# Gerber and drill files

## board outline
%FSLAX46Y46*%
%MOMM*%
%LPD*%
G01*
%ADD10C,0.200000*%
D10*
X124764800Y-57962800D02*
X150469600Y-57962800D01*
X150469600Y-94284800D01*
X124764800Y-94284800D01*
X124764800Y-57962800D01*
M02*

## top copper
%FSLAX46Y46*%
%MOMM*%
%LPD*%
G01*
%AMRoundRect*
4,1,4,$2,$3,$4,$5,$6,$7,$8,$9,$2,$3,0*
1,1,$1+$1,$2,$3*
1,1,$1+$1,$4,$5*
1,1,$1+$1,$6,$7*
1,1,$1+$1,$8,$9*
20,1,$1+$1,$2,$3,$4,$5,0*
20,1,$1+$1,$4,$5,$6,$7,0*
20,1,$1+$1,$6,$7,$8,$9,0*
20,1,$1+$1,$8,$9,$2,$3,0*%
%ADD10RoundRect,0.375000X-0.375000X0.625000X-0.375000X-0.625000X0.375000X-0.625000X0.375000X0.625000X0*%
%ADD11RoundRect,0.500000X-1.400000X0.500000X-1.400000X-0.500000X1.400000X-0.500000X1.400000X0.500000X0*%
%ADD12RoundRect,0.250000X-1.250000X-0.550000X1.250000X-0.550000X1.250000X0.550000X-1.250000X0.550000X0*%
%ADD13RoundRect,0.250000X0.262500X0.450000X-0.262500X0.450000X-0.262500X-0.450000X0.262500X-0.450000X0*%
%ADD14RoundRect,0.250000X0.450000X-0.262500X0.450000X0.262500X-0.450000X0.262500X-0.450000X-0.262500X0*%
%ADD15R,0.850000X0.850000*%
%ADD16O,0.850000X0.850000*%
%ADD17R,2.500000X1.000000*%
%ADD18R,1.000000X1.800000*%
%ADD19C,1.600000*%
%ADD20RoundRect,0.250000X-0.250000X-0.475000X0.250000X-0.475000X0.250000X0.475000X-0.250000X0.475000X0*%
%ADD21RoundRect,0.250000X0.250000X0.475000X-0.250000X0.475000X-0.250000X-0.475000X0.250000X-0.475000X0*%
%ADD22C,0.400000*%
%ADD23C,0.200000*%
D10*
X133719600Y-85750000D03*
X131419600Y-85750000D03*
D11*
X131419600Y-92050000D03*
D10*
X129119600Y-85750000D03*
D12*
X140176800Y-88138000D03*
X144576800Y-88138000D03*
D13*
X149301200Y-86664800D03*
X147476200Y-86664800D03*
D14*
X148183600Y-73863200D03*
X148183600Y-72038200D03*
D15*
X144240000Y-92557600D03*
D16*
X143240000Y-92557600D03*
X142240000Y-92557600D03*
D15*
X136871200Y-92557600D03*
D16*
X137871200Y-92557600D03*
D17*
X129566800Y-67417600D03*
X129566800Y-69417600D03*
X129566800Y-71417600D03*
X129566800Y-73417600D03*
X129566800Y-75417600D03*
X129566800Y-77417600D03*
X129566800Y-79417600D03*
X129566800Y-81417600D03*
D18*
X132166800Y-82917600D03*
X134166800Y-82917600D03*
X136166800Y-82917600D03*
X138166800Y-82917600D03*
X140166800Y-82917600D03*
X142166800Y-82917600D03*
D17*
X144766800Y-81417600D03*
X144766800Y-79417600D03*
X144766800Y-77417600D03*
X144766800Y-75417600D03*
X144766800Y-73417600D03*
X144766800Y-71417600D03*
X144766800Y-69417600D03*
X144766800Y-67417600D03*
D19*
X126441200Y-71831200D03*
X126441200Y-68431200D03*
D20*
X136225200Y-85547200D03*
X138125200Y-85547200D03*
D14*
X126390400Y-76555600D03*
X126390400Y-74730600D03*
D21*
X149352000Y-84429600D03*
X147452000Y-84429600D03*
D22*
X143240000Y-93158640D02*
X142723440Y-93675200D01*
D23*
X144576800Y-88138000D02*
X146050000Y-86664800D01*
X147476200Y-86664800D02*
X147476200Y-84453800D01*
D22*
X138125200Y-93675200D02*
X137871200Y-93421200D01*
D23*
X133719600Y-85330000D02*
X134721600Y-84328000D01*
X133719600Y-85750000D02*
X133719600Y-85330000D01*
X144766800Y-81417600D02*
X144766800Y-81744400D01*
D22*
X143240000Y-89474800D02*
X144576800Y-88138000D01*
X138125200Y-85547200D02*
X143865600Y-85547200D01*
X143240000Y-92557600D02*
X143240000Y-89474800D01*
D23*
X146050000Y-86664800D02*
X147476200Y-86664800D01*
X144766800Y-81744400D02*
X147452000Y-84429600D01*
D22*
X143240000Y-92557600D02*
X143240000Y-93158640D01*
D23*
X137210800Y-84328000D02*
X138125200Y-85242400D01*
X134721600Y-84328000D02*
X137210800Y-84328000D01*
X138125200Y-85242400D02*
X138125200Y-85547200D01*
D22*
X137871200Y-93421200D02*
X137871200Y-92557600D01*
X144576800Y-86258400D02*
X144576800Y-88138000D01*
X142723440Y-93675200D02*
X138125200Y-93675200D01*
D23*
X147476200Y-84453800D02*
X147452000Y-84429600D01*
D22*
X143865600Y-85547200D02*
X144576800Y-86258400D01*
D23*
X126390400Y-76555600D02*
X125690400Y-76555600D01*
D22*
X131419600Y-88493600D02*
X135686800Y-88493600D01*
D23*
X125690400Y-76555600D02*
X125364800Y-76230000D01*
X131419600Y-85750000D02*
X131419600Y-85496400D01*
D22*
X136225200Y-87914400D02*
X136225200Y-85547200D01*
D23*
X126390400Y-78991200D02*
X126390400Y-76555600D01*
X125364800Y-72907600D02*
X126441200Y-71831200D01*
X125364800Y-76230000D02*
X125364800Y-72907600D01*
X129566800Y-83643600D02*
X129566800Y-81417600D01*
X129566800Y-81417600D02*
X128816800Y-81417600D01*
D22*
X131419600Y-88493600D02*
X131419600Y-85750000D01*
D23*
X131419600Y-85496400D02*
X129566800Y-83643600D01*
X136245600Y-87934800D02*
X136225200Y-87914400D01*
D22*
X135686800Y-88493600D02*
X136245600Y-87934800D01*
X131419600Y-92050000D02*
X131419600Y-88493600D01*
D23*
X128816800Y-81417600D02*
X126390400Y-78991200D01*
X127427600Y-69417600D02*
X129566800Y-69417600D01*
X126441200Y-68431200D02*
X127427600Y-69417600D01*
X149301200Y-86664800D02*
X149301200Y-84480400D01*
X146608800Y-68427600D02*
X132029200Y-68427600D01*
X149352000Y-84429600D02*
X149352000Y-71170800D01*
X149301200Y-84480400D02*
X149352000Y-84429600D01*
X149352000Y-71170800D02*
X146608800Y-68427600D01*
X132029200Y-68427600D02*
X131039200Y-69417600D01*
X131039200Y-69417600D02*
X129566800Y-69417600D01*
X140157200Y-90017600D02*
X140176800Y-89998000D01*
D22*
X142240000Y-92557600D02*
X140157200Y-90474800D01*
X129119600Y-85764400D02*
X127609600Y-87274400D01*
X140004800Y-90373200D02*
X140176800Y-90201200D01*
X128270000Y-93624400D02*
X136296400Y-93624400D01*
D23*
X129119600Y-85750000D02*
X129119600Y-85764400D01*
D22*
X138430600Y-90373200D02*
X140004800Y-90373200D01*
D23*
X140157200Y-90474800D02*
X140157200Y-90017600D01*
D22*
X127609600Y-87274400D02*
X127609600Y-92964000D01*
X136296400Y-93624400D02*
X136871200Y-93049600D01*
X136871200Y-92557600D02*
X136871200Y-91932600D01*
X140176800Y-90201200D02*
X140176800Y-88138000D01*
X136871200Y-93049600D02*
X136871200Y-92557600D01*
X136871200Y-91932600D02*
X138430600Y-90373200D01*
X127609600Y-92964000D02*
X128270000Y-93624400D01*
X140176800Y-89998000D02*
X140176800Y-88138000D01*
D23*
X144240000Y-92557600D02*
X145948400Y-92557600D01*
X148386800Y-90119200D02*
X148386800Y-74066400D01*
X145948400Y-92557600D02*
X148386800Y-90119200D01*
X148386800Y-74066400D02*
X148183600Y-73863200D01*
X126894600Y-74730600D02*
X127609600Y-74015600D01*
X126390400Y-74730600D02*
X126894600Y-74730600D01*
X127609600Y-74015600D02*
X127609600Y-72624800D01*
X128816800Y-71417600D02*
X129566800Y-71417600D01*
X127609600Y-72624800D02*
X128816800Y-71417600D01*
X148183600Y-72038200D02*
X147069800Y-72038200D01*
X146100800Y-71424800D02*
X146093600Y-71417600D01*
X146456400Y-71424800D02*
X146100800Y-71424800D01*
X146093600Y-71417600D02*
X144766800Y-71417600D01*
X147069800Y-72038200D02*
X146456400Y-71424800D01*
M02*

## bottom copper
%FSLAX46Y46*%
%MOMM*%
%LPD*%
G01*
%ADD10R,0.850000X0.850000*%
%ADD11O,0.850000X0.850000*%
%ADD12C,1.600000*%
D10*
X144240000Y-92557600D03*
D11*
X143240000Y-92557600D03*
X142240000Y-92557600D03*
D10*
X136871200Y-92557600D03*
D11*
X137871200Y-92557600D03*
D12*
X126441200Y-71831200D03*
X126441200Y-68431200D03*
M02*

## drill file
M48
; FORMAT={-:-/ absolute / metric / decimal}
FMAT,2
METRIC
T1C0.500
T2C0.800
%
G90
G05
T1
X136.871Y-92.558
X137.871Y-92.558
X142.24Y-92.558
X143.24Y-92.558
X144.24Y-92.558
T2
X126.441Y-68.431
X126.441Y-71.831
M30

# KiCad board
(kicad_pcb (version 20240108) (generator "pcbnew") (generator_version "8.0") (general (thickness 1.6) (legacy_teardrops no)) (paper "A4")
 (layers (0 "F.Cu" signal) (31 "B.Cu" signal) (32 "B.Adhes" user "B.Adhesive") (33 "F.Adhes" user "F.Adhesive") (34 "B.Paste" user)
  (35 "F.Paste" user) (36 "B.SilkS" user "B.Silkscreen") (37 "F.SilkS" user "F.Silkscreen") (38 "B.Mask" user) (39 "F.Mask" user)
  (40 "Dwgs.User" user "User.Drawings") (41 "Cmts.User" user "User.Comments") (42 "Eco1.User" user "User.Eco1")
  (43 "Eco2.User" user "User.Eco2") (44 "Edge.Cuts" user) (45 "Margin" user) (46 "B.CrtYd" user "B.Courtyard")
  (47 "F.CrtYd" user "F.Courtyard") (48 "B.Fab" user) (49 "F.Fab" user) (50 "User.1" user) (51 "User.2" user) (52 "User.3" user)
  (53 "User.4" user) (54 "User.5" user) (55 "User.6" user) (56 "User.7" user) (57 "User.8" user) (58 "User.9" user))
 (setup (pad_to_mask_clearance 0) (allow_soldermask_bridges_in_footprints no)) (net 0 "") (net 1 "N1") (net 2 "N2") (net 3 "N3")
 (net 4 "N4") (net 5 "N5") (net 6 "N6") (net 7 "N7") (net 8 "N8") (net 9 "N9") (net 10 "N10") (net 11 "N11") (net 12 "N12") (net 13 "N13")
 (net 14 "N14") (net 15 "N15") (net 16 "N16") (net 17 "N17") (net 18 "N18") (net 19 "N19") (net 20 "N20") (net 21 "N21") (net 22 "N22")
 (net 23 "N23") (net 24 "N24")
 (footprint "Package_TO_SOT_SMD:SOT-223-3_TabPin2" (layer "F.Cu") (at 131.4196 88.9 -90)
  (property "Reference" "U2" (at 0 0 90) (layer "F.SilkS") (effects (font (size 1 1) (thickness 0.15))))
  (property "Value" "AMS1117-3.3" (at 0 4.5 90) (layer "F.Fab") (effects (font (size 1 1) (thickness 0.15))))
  (pad "1" smd roundrect (at -3.15 -2.3 270) (size 2 1.5) (layers "F.Cu" "F.Paste" "F.Mask") (roundrect_rratio 0.25) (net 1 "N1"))
  (pad "2" smd roundrect (at -3.15 0 270) (size 2 1.5) (layers "F.Cu" "F.Paste" "F.Mask") (roundrect_rratio 0.25) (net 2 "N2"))
  (pad "2" smd roundrect (at 3.15 0 270) (size 2 3.8) (layers "F.Cu" "F.Paste" "F.Mask") (roundrect_rratio 0.25) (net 2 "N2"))
  (pad "3" smd roundrect (at -3.15 2.3 270) (size 2 1.5) (layers "F.Cu" "F.Paste" "F.Mask") (roundrect_rratio 0.25) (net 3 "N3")))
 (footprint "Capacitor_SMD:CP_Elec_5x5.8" (layer "F.Cu") (at 142.3768 88.138)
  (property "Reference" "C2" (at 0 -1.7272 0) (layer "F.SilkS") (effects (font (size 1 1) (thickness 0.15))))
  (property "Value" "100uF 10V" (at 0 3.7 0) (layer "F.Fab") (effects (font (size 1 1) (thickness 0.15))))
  (pad "1" smd roundrect (at -2.2 0) (size 3 1.6) (layers "F.Cu" "F.Paste" "F.Mask") (roundrect_rratio 0.15625) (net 3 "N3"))
  (pad "2" smd roundrect (at 2.2 0) (size 3 1.6) (layers "F.Cu" "F.Paste" "F.Mask") (roundrect_rratio 0.15625) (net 1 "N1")))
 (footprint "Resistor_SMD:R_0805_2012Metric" (layer "F.Cu") (at 148.3887 86.6648 180)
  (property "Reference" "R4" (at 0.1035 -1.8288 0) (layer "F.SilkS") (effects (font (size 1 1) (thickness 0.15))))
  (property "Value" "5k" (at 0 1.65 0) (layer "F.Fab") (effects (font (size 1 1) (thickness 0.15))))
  (pad "1" smd roundrect (at -0.9125 0 180) (size 1.025 1.4) (layers "F.Cu" "F.Paste" "F.Mask") (roundrect_rratio 0.243902) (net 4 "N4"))
  (pad "2" smd roundrect (at 0.9125 0 180) (size 1.025 1.4) (layers "F.Cu" "F.Paste" "F.Mask") (roundrect_rratio 0.243902) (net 1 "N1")))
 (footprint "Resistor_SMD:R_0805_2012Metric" (layer "F.Cu") (at 148.1836 72.9507 90)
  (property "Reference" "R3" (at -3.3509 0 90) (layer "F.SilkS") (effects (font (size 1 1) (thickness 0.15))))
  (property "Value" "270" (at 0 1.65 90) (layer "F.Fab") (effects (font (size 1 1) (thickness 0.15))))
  (pad "1" smd roundrect (at -0.9125 0 90) (size 1.025 1.4) (layers "F.Cu" "F.Paste" "F.Mask") (roundrect_rratio 0.243902) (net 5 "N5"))
  (pad "2" smd roundrect (at 0.9125 0 90) (size 1.025 1.4) (layers "F.Cu" "F.Paste" "F.Mask") (roundrect_rratio 0.243902) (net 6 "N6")))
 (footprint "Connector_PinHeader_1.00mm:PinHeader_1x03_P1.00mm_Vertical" (layer "F.Cu") (at 144.24 92.5576 -90)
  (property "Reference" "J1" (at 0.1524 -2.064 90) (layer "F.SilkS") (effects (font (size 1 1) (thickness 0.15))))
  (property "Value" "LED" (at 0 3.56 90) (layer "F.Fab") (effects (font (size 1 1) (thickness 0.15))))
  (pad "1" thru_hole rect (at 0 0 270) (size 0.85 0.85) (drill 0.5) (layers "*.Cu" "*.Mask") (remove_unused_layers no) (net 5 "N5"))
  (pad "2" thru_hole oval (at 0 1 270) (size 0.85 0.85) (drill 0.5) (layers "*.Cu" "*.Mask") (remove_unused_layers no) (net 1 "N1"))
  (pad "3" thru_hole oval (at 0 2 270) (size 0.85 0.85) (drill 0.5) (layers "*.Cu" "*.Mask") (remove_unused_layers no) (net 3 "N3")))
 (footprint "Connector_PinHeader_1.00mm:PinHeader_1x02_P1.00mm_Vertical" (layer "F.Cu") (at 136.8712 92.5576 90)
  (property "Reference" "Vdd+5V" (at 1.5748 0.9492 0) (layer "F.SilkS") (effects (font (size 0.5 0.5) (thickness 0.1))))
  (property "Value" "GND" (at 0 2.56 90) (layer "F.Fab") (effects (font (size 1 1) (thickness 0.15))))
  (pad "1" thru_hole rect (at 0 0 90) (size 0.85 0.85) (drill 0.5) (layers "*.Cu" "*.Mask") (remove_unused_layers no) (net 3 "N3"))
  (pad "2" thru_hole oval (at 0 1 90) (size 0.85 0.85) (drill 0.5) (layers "*.Cu" "*.Mask") (remove_unused_layers no) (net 1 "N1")))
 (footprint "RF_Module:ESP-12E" (layer "F.Cu") (at 137.1668 70.9176)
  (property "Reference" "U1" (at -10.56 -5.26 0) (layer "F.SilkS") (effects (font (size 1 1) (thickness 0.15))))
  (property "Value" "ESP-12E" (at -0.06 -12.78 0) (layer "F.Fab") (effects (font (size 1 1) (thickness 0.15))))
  (pad "1" smd rect (at -7.6 -3.5) (size 2.5 1) (layers "F.Cu" "F.Paste" "F.Mask") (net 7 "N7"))
  (pad "2" smd rect (at -7.6 -1.5) (size 2.5 1) (layers "F.Cu" "F.Paste" "F.Mask") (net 4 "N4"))
  (pad "3" smd rect (at -7.6 0.5) (size 2.5 1) (layers "F.Cu" "F.Paste" "F.Mask") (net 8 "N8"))
  (pad "4" smd rect (at -7.6 2.5) (size 2.5 1) (layers "F.Cu" "F.Paste" "F.Mask") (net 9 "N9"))
  (pad "5" smd rect (at -7.6 4.5) (size 2.5 1) (layers "F.Cu" "F.Paste" "F.Mask") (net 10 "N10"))
  (pad "6" smd rect (at -7.6 6.5) (size 2.5 1) (layers "F.Cu" "F.Paste" "F.Mask") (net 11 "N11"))
  (pad "7" smd rect (at -7.6 8.5) (size 2.5 1) (layers "F.Cu" "F.Paste" "F.Mask") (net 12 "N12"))
  (pad "8" smd rect (at -7.6 10.5) (size 2.5 1) (layers "F.Cu" "F.Paste" "F.Mask") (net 2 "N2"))
  (pad "9" smd rect (at -5 12) (size 1 1.8) (layers "F.Cu" "F.Paste" "F.Mask") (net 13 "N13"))
  (pad "10" smd rect (at -3 12) (size 1 1.8) (layers "F.Cu" "F.Paste" "F.Mask") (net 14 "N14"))
  (pad "11" smd rect (at -1 12) (size 1 1.8) (layers "F.Cu" "F.Paste" "F.Mask") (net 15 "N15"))
  (pad "12" smd rect (at 1 12) (size 1 1.8) (layers "F.Cu" "F.Paste" "F.Mask") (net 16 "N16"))
  (pad "13" smd rect (at 3 12) (size 1 1.8) (layers "F.Cu" "F.Paste" "F.Mask") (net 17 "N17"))
  (pad "14" smd rect (at 5 12) (size 1 1.8) (layers "F.Cu" "F.Paste" "F.Mask") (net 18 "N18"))
  (pad "15" smd rect (at 7.6 10.5) (size 2.5 1) (layers "F.Cu" "F.Paste" "F.Mask") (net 1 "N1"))
  (pad "16" smd rect (at 7.6 8.5) (size 2.5 1) (layers "F.Cu" "F.Paste" "F.Mask") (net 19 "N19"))
  (pad "17" smd rect (at 7.6 6.5) (size 2.5 1) (layers "F.Cu" "F.Paste" "F.Mask") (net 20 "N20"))
  (pad "18" smd rect (at 7.6 4.5) (size 2.5 1) (layers "F.Cu" "F.Paste" "F.Mask") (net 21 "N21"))
  (pad "19" smd rect (at 7.6 2.5) (size 2.5 1) (layers "F.Cu" "F.Paste" "F.Mask") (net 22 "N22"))
  (pad "20" smd rect (at 7.6 0.5) (size 2.5 1) (layers "F.Cu" "F.Paste" "F.Mask") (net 6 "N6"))
  (pad "21" smd rect (at 7.6 -1.5) (size 2.5 1) (layers "F.Cu" "F.Paste" "F.Mask") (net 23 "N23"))
  (pad "22" smd rect (at 7.6 -3.5) (size 2.5 1) (layers "F.Cu" "F.Paste" "F.Mask") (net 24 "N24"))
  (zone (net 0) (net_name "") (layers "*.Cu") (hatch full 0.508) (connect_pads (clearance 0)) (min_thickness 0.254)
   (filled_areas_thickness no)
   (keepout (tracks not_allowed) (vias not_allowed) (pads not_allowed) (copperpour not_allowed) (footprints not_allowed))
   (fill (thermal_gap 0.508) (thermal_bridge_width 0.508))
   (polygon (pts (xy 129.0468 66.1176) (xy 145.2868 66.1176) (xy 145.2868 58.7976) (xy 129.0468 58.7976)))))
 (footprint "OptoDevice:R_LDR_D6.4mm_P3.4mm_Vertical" (layer "F.Cu") (at 126.4412 71.8312 90)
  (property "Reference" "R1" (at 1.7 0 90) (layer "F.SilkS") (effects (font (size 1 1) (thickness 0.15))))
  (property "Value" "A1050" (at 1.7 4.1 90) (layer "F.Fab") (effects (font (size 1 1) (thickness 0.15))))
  (pad "1" thru_hole circle (at 0 0 90) (size 1.6 1.6) (drill 0.8) (layers "*.Cu" "*.Mask") (remove_unused_layers no) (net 2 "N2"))
  (pad "2" thru_hole circle (at 3.4 0 90) (size 1.6 1.6) (drill 0.8) (layers "*.Cu" "*.Mask") (remove_unused_layers no) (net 4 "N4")))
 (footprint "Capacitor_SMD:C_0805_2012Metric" (layer "F.Cu") (at 137.1752 85.5472)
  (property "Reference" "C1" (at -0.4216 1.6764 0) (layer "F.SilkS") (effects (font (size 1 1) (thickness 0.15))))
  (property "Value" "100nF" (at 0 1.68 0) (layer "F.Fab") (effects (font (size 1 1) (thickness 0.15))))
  (pad "1" smd roundrect (at -0.95 0) (size 1 1.45) (layers "F.Cu" "F.Paste" "F.Mask") (roundrect_rratio 0.25) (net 2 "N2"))
  (pad "2" smd roundrect (at 0.95 0) (size 1 1.45) (layers "F.Cu" "F.Paste" "F.Mask") (roundrect_rratio 0.25) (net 1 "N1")))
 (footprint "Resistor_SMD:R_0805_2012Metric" (layer "F.Cu") (at 126.3904 75.6431 90)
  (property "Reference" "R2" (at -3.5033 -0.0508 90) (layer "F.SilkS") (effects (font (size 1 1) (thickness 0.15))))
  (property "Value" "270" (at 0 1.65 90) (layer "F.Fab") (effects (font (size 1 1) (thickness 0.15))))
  (pad "1" smd roundrect (at -0.9125 0 90) (size 1.025 1.4) (layers "F.Cu" "F.Paste" "F.Mask") (roundrect_rratio 0.243902) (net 2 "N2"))
  (pad "2" smd roundrect (at 0.9125 0 90) (size 1.025 1.4) (layers "F.Cu" "F.Paste" "F.Mask") (roundrect_rratio 0.243902) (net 8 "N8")))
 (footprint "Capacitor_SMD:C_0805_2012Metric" (layer "F.Cu") (at 148.402 84.4296 180)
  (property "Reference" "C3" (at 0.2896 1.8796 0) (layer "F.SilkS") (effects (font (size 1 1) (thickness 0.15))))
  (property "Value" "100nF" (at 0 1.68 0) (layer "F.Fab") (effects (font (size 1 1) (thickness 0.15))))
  (pad "1" smd roundrect (at -0.95 0 180) (size 1 1.45) (layers "F.Cu" "F.Paste" "F.Mask") (roundrect_rratio 0.25) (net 4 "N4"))
  (pad "2" smd roundrect (at 0.95 0 180) (size 1 1.45) (layers "F.Cu" "F.Paste" "F.Mask") (roundrect_rratio 0.25) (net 1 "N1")))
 (gr_rect (start 124.7648 57.9628) (end 150.4696 94.2848) (stroke (width 0.2) (type default)) (fill none) (layer "Edge.Cuts"))
 (segment (start 143.24 93.15864) (end 142.72344 93.6752) (width 0.4) (layer "F.Cu") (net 1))
 (segment (start 144.5768 88.138) (end 146.05 86.6648) (width 0.2) (layer "F.Cu") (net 1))
 (segment (start 147.4762 86.6648) (end 147.4762 84.4538) (width 0.2) (layer "F.Cu") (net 1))
 (segment (start 138.1252 93.6752) (end 137.8712 93.4212) (width 0.4) (layer "F.Cu") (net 1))
 (segment (start 133.7196 85.33) (end 134.7216 84.328) (width 0.2) (layer "F.Cu") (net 1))
 (segment (start 133.7196 85.75) (end 133.7196 85.33) (width 0.2) (layer "F.Cu") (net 1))
 (segment (start 144.7668 81.4176) (end 144.7668 81.7444) (width 0.2) (layer "F.Cu") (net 1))
 (segment (start 143.24 89.4748) (end 144.5768 88.138) (width 0.4) (layer "F.Cu") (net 1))
 (segment (start 138.1252 85.5472) (end 143.8656 85.5472) (width 0.4) (layer "F.Cu") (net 1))
 (segment (start 143.24 92.5576) (end 143.24 89.4748) (width 0.4) (layer "F.Cu") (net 1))
 (segment (start 146.05 86.6648) (end 147.4762 86.6648) (width 0.2) (layer "F.Cu") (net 1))
 (segment (start 144.7668 81.7444) (end 147.452 84.4296) (width 0.2) (layer "F.Cu") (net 1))
 (segment (start 143.24 92.5576) (end 143.24 93.15864) (width 0.4) (layer "F.Cu") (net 1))
 (segment (start 137.2108 84.328) (end 138.1252 85.2424) (width 0.2) (layer "F.Cu") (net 1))
 (segment (start 134.7216 84.328) (end 137.2108 84.328) (width 0.2) (layer "F.Cu") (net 1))
 (segment (start 138.1252 85.2424) (end 138.1252 85.5472) (width 0.2) (layer "F.Cu") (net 1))
 (segment (start 137.8712 93.4212) (end 137.8712 92.5576) (width 0.4) (layer "F.Cu") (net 1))
 (segment (start 144.5768 86.2584) (end 144.5768 88.138) (width 0.4) (layer "F.Cu") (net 1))
 (segment (start 142.72344 93.6752) (end 138.1252 93.6752) (width 0.4) (layer "F.Cu") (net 1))
 (segment (start 147.4762 84.4538) (end 147.452 84.4296) (width 0.2) (layer "F.Cu") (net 1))
 (segment (start 143.8656 85.5472) (end 144.5768 86.2584) (width 0.4) (layer "F.Cu") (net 1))
 (segment (start 126.3904 76.5556) (end 125.6904 76.5556) (width 0.2) (layer "F.Cu") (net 2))
 (segment (start 131.4196 88.4936) (end 135.6868 88.4936) (width 0.4) (layer "F.Cu") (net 2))
 (segment (start 125.6904 76.5556) (end 125.3648 76.23) (width 0.2) (layer "F.Cu") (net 2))
 (segment (start 131.4196 85.75) (end 131.4196 85.4964) (width 0.2) (layer "F.Cu") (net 2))
 (segment (start 136.2252 87.9144) (end 136.2252 85.5472) (width 0.4) (layer "F.Cu") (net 2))
 (segment (start 126.3904 78.9912) (end 126.3904 76.5556) (width 0.2) (layer "F.Cu") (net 2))
 (segment (start 125.3648 72.9076) (end 126.4412 71.8312) (width 0.2) (layer "F.Cu") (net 2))
 (segment (start 125.3648 76.23) (end 125.3648 72.9076) (width 0.2) (layer "F.Cu") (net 2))
 (segment (start 129.5668 83.6436) (end 129.5668 81.4176) (width 0.2) (layer "F.Cu") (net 2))
 (segment (start 129.5668 81.4176) (end 128.8168 81.4176) (width 0.2) (layer "F.Cu") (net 2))
 (segment (start 131.4196 88.4936) (end 131.4196 85.75) (width 0.4) (layer "F.Cu") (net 2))
 (segment (start 131.4196 85.4964) (end 129.5668 83.6436) (width 0.2) (layer "F.Cu") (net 2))
 (segment (start 136.2456 87.9348) (end 136.2252 87.9144) (width 0.2) (layer "F.Cu") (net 2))
 (segment (start 135.6868 88.4936) (end 136.2456 87.9348) (width 0.4) (layer "F.Cu") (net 2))
 (segment (start 131.4196 92.05) (end 131.4196 88.4936) (width 0.4) (layer "F.Cu") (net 2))
 (segment (start 128.8168 81.4176) (end 126.3904 78.9912) (width 0.2) (layer "F.Cu") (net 2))
 (segment (start 127.4276 69.4176) (end 129.5668 69.4176) (width 0.2) (layer "F.Cu") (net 4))
 (segment (start 126.4412 68.4312) (end 127.4276 69.4176) (width 0.2) (layer "F.Cu") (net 4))
 (segment (start 149.3012 86.6648) (end 149.3012 84.4804) (width 0.2) (layer "F.Cu") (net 4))
 (segment (start 146.6088 68.4276) (end 132.0292 68.4276) (width 0.2) (layer "F.Cu") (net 4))
 (segment (start 149.352 84.4296) (end 149.352 71.1708) (width 0.2) (layer "F.Cu") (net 4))
 (segment (start 149.3012 84.4804) (end 149.352 84.4296) (width 0.2) (layer "F.Cu") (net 4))
 (segment (start 149.352 71.1708) (end 146.6088 68.4276) (width 0.2) (layer "F.Cu") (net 4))
 (segment (start 132.0292 68.4276) (end 131.0392 69.4176) (width 0.2) (layer "F.Cu") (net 4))
 (segment (start 131.0392 69.4176) (end 129.5668 69.4176) (width 0.2) (layer "F.Cu") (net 4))
 (segment (start 140.1572 90.0176) (end 140.1768 89.998) (width 0.2) (layer "F.Cu") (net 3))
 (segment (start 142.24 92.5576) (end 140.1572 90.4748) (width 0.4) (layer "F.Cu") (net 3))
 (segment (start 129.1196 85.7644) (end 127.6096 87.2744) (width 0.4) (layer "F.Cu") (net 3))
 (segment (start 140.0048 90.3732) (end 140.1768 90.2012) (width 0.4) (layer "F.Cu") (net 3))
 (segment (start 128.27 93.6244) (end 136.2964 93.6244) (width 0.4) (layer "F.Cu") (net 3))
 (segment (start 129.1196 85.75) (end 129.1196 85.7644) (width 0.2) (layer "F.Cu") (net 3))
 (segment (start 138.4306 90.3732) (end 140.0048 90.3732) (width 0.4) (layer "F.Cu") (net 3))
 (segment (start 140.1572 90.4748) (end 140.1572 90.0176) (width 0.2) (layer "F.Cu") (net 3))
 (segment (start 127.6096 87.2744) (end 127.6096 92.964) (width 0.4) (layer "F.Cu") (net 3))
 (segment (start 136.2964 93.6244) (end 136.8712 93.0496) (width 0.4) (layer "F.Cu") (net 3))
 (segment (start 136.8712 92.5576) (end 136.8712 91.9326) (width 0.4) (layer "F.Cu") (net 3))
 (segment (start 140.1768 90.2012) (end 140.1768 88.138) (width 0.4) (layer "F.Cu") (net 3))
 (segment (start 136.8712 93.0496) (end 136.8712 92.5576) (width 0.4) (layer "F.Cu") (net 3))
 (segment (start 136.8712 91.9326) (end 138.4306 90.3732) (width 0.4) (layer "F.Cu") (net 3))
 (segment (start 127.6096 92.964) (end 128.27 93.6244) (width 0.4) (layer "F.Cu") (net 3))
 (segment (start 140.1768 89.998) (end 140.1768 88.138) (width 0.4) (layer "F.Cu") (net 3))
 (segment (start 144.24 92.5576) (end 145.9484 92.5576) (width 0.2) (layer "F.Cu") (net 5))
 (segment (start 148.3868 90.1192) (end 148.3868 74.0664) (width 0.2) (layer "F.Cu") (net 5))
 (segment (start 145.9484 92.5576) (end 148.3868 90.1192) (width 0.2) (layer "F.Cu") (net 5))
 (segment (start 148.3868 74.0664) (end 148.1836 73.8632) (width 0.2) (layer "F.Cu") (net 5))
 (segment (start 126.8946 74.7306) (end 127.6096 74.0156) (width 0.2) (layer "F.Cu") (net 8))
 (segment (start 126.3904 74.7306) (end 126.8946 74.7306) (width 0.2) (layer "F.Cu") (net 8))
 (segment (start 127.6096 74.0156) (end 127.6096 72.6248) (width 0.2) (layer "F.Cu") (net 8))
 (segment (start 128.8168 71.4176) (end 129.5668 71.4176) (width 0.2) (layer "F.Cu") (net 8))
 (segment (start 127.6096 72.6248) (end 128.8168 71.4176) (width 0.2) (layer "F.Cu") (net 8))
 (segment (start 148.1836 72.0382) (end 147.0698 72.0382) (width 0.2) (layer "F.Cu") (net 6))
 (segment (start 146.1008 71.4248) (end 146.0936 71.4176) (width 0.2) (layer "F.Cu") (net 6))
 (segment (start 146.4564 71.4248) (end 146.1008 71.4248) (width 0.2) (layer "F.Cu") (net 6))
 (segment (start 146.0936 71.4176) (end 144.7668 71.4176) (width 0.2) (layer "F.Cu") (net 6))
 (segment (start 147.0698 72.0382) (end 146.4564 71.4248) (width 0.2) (layer "F.Cu") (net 6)))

